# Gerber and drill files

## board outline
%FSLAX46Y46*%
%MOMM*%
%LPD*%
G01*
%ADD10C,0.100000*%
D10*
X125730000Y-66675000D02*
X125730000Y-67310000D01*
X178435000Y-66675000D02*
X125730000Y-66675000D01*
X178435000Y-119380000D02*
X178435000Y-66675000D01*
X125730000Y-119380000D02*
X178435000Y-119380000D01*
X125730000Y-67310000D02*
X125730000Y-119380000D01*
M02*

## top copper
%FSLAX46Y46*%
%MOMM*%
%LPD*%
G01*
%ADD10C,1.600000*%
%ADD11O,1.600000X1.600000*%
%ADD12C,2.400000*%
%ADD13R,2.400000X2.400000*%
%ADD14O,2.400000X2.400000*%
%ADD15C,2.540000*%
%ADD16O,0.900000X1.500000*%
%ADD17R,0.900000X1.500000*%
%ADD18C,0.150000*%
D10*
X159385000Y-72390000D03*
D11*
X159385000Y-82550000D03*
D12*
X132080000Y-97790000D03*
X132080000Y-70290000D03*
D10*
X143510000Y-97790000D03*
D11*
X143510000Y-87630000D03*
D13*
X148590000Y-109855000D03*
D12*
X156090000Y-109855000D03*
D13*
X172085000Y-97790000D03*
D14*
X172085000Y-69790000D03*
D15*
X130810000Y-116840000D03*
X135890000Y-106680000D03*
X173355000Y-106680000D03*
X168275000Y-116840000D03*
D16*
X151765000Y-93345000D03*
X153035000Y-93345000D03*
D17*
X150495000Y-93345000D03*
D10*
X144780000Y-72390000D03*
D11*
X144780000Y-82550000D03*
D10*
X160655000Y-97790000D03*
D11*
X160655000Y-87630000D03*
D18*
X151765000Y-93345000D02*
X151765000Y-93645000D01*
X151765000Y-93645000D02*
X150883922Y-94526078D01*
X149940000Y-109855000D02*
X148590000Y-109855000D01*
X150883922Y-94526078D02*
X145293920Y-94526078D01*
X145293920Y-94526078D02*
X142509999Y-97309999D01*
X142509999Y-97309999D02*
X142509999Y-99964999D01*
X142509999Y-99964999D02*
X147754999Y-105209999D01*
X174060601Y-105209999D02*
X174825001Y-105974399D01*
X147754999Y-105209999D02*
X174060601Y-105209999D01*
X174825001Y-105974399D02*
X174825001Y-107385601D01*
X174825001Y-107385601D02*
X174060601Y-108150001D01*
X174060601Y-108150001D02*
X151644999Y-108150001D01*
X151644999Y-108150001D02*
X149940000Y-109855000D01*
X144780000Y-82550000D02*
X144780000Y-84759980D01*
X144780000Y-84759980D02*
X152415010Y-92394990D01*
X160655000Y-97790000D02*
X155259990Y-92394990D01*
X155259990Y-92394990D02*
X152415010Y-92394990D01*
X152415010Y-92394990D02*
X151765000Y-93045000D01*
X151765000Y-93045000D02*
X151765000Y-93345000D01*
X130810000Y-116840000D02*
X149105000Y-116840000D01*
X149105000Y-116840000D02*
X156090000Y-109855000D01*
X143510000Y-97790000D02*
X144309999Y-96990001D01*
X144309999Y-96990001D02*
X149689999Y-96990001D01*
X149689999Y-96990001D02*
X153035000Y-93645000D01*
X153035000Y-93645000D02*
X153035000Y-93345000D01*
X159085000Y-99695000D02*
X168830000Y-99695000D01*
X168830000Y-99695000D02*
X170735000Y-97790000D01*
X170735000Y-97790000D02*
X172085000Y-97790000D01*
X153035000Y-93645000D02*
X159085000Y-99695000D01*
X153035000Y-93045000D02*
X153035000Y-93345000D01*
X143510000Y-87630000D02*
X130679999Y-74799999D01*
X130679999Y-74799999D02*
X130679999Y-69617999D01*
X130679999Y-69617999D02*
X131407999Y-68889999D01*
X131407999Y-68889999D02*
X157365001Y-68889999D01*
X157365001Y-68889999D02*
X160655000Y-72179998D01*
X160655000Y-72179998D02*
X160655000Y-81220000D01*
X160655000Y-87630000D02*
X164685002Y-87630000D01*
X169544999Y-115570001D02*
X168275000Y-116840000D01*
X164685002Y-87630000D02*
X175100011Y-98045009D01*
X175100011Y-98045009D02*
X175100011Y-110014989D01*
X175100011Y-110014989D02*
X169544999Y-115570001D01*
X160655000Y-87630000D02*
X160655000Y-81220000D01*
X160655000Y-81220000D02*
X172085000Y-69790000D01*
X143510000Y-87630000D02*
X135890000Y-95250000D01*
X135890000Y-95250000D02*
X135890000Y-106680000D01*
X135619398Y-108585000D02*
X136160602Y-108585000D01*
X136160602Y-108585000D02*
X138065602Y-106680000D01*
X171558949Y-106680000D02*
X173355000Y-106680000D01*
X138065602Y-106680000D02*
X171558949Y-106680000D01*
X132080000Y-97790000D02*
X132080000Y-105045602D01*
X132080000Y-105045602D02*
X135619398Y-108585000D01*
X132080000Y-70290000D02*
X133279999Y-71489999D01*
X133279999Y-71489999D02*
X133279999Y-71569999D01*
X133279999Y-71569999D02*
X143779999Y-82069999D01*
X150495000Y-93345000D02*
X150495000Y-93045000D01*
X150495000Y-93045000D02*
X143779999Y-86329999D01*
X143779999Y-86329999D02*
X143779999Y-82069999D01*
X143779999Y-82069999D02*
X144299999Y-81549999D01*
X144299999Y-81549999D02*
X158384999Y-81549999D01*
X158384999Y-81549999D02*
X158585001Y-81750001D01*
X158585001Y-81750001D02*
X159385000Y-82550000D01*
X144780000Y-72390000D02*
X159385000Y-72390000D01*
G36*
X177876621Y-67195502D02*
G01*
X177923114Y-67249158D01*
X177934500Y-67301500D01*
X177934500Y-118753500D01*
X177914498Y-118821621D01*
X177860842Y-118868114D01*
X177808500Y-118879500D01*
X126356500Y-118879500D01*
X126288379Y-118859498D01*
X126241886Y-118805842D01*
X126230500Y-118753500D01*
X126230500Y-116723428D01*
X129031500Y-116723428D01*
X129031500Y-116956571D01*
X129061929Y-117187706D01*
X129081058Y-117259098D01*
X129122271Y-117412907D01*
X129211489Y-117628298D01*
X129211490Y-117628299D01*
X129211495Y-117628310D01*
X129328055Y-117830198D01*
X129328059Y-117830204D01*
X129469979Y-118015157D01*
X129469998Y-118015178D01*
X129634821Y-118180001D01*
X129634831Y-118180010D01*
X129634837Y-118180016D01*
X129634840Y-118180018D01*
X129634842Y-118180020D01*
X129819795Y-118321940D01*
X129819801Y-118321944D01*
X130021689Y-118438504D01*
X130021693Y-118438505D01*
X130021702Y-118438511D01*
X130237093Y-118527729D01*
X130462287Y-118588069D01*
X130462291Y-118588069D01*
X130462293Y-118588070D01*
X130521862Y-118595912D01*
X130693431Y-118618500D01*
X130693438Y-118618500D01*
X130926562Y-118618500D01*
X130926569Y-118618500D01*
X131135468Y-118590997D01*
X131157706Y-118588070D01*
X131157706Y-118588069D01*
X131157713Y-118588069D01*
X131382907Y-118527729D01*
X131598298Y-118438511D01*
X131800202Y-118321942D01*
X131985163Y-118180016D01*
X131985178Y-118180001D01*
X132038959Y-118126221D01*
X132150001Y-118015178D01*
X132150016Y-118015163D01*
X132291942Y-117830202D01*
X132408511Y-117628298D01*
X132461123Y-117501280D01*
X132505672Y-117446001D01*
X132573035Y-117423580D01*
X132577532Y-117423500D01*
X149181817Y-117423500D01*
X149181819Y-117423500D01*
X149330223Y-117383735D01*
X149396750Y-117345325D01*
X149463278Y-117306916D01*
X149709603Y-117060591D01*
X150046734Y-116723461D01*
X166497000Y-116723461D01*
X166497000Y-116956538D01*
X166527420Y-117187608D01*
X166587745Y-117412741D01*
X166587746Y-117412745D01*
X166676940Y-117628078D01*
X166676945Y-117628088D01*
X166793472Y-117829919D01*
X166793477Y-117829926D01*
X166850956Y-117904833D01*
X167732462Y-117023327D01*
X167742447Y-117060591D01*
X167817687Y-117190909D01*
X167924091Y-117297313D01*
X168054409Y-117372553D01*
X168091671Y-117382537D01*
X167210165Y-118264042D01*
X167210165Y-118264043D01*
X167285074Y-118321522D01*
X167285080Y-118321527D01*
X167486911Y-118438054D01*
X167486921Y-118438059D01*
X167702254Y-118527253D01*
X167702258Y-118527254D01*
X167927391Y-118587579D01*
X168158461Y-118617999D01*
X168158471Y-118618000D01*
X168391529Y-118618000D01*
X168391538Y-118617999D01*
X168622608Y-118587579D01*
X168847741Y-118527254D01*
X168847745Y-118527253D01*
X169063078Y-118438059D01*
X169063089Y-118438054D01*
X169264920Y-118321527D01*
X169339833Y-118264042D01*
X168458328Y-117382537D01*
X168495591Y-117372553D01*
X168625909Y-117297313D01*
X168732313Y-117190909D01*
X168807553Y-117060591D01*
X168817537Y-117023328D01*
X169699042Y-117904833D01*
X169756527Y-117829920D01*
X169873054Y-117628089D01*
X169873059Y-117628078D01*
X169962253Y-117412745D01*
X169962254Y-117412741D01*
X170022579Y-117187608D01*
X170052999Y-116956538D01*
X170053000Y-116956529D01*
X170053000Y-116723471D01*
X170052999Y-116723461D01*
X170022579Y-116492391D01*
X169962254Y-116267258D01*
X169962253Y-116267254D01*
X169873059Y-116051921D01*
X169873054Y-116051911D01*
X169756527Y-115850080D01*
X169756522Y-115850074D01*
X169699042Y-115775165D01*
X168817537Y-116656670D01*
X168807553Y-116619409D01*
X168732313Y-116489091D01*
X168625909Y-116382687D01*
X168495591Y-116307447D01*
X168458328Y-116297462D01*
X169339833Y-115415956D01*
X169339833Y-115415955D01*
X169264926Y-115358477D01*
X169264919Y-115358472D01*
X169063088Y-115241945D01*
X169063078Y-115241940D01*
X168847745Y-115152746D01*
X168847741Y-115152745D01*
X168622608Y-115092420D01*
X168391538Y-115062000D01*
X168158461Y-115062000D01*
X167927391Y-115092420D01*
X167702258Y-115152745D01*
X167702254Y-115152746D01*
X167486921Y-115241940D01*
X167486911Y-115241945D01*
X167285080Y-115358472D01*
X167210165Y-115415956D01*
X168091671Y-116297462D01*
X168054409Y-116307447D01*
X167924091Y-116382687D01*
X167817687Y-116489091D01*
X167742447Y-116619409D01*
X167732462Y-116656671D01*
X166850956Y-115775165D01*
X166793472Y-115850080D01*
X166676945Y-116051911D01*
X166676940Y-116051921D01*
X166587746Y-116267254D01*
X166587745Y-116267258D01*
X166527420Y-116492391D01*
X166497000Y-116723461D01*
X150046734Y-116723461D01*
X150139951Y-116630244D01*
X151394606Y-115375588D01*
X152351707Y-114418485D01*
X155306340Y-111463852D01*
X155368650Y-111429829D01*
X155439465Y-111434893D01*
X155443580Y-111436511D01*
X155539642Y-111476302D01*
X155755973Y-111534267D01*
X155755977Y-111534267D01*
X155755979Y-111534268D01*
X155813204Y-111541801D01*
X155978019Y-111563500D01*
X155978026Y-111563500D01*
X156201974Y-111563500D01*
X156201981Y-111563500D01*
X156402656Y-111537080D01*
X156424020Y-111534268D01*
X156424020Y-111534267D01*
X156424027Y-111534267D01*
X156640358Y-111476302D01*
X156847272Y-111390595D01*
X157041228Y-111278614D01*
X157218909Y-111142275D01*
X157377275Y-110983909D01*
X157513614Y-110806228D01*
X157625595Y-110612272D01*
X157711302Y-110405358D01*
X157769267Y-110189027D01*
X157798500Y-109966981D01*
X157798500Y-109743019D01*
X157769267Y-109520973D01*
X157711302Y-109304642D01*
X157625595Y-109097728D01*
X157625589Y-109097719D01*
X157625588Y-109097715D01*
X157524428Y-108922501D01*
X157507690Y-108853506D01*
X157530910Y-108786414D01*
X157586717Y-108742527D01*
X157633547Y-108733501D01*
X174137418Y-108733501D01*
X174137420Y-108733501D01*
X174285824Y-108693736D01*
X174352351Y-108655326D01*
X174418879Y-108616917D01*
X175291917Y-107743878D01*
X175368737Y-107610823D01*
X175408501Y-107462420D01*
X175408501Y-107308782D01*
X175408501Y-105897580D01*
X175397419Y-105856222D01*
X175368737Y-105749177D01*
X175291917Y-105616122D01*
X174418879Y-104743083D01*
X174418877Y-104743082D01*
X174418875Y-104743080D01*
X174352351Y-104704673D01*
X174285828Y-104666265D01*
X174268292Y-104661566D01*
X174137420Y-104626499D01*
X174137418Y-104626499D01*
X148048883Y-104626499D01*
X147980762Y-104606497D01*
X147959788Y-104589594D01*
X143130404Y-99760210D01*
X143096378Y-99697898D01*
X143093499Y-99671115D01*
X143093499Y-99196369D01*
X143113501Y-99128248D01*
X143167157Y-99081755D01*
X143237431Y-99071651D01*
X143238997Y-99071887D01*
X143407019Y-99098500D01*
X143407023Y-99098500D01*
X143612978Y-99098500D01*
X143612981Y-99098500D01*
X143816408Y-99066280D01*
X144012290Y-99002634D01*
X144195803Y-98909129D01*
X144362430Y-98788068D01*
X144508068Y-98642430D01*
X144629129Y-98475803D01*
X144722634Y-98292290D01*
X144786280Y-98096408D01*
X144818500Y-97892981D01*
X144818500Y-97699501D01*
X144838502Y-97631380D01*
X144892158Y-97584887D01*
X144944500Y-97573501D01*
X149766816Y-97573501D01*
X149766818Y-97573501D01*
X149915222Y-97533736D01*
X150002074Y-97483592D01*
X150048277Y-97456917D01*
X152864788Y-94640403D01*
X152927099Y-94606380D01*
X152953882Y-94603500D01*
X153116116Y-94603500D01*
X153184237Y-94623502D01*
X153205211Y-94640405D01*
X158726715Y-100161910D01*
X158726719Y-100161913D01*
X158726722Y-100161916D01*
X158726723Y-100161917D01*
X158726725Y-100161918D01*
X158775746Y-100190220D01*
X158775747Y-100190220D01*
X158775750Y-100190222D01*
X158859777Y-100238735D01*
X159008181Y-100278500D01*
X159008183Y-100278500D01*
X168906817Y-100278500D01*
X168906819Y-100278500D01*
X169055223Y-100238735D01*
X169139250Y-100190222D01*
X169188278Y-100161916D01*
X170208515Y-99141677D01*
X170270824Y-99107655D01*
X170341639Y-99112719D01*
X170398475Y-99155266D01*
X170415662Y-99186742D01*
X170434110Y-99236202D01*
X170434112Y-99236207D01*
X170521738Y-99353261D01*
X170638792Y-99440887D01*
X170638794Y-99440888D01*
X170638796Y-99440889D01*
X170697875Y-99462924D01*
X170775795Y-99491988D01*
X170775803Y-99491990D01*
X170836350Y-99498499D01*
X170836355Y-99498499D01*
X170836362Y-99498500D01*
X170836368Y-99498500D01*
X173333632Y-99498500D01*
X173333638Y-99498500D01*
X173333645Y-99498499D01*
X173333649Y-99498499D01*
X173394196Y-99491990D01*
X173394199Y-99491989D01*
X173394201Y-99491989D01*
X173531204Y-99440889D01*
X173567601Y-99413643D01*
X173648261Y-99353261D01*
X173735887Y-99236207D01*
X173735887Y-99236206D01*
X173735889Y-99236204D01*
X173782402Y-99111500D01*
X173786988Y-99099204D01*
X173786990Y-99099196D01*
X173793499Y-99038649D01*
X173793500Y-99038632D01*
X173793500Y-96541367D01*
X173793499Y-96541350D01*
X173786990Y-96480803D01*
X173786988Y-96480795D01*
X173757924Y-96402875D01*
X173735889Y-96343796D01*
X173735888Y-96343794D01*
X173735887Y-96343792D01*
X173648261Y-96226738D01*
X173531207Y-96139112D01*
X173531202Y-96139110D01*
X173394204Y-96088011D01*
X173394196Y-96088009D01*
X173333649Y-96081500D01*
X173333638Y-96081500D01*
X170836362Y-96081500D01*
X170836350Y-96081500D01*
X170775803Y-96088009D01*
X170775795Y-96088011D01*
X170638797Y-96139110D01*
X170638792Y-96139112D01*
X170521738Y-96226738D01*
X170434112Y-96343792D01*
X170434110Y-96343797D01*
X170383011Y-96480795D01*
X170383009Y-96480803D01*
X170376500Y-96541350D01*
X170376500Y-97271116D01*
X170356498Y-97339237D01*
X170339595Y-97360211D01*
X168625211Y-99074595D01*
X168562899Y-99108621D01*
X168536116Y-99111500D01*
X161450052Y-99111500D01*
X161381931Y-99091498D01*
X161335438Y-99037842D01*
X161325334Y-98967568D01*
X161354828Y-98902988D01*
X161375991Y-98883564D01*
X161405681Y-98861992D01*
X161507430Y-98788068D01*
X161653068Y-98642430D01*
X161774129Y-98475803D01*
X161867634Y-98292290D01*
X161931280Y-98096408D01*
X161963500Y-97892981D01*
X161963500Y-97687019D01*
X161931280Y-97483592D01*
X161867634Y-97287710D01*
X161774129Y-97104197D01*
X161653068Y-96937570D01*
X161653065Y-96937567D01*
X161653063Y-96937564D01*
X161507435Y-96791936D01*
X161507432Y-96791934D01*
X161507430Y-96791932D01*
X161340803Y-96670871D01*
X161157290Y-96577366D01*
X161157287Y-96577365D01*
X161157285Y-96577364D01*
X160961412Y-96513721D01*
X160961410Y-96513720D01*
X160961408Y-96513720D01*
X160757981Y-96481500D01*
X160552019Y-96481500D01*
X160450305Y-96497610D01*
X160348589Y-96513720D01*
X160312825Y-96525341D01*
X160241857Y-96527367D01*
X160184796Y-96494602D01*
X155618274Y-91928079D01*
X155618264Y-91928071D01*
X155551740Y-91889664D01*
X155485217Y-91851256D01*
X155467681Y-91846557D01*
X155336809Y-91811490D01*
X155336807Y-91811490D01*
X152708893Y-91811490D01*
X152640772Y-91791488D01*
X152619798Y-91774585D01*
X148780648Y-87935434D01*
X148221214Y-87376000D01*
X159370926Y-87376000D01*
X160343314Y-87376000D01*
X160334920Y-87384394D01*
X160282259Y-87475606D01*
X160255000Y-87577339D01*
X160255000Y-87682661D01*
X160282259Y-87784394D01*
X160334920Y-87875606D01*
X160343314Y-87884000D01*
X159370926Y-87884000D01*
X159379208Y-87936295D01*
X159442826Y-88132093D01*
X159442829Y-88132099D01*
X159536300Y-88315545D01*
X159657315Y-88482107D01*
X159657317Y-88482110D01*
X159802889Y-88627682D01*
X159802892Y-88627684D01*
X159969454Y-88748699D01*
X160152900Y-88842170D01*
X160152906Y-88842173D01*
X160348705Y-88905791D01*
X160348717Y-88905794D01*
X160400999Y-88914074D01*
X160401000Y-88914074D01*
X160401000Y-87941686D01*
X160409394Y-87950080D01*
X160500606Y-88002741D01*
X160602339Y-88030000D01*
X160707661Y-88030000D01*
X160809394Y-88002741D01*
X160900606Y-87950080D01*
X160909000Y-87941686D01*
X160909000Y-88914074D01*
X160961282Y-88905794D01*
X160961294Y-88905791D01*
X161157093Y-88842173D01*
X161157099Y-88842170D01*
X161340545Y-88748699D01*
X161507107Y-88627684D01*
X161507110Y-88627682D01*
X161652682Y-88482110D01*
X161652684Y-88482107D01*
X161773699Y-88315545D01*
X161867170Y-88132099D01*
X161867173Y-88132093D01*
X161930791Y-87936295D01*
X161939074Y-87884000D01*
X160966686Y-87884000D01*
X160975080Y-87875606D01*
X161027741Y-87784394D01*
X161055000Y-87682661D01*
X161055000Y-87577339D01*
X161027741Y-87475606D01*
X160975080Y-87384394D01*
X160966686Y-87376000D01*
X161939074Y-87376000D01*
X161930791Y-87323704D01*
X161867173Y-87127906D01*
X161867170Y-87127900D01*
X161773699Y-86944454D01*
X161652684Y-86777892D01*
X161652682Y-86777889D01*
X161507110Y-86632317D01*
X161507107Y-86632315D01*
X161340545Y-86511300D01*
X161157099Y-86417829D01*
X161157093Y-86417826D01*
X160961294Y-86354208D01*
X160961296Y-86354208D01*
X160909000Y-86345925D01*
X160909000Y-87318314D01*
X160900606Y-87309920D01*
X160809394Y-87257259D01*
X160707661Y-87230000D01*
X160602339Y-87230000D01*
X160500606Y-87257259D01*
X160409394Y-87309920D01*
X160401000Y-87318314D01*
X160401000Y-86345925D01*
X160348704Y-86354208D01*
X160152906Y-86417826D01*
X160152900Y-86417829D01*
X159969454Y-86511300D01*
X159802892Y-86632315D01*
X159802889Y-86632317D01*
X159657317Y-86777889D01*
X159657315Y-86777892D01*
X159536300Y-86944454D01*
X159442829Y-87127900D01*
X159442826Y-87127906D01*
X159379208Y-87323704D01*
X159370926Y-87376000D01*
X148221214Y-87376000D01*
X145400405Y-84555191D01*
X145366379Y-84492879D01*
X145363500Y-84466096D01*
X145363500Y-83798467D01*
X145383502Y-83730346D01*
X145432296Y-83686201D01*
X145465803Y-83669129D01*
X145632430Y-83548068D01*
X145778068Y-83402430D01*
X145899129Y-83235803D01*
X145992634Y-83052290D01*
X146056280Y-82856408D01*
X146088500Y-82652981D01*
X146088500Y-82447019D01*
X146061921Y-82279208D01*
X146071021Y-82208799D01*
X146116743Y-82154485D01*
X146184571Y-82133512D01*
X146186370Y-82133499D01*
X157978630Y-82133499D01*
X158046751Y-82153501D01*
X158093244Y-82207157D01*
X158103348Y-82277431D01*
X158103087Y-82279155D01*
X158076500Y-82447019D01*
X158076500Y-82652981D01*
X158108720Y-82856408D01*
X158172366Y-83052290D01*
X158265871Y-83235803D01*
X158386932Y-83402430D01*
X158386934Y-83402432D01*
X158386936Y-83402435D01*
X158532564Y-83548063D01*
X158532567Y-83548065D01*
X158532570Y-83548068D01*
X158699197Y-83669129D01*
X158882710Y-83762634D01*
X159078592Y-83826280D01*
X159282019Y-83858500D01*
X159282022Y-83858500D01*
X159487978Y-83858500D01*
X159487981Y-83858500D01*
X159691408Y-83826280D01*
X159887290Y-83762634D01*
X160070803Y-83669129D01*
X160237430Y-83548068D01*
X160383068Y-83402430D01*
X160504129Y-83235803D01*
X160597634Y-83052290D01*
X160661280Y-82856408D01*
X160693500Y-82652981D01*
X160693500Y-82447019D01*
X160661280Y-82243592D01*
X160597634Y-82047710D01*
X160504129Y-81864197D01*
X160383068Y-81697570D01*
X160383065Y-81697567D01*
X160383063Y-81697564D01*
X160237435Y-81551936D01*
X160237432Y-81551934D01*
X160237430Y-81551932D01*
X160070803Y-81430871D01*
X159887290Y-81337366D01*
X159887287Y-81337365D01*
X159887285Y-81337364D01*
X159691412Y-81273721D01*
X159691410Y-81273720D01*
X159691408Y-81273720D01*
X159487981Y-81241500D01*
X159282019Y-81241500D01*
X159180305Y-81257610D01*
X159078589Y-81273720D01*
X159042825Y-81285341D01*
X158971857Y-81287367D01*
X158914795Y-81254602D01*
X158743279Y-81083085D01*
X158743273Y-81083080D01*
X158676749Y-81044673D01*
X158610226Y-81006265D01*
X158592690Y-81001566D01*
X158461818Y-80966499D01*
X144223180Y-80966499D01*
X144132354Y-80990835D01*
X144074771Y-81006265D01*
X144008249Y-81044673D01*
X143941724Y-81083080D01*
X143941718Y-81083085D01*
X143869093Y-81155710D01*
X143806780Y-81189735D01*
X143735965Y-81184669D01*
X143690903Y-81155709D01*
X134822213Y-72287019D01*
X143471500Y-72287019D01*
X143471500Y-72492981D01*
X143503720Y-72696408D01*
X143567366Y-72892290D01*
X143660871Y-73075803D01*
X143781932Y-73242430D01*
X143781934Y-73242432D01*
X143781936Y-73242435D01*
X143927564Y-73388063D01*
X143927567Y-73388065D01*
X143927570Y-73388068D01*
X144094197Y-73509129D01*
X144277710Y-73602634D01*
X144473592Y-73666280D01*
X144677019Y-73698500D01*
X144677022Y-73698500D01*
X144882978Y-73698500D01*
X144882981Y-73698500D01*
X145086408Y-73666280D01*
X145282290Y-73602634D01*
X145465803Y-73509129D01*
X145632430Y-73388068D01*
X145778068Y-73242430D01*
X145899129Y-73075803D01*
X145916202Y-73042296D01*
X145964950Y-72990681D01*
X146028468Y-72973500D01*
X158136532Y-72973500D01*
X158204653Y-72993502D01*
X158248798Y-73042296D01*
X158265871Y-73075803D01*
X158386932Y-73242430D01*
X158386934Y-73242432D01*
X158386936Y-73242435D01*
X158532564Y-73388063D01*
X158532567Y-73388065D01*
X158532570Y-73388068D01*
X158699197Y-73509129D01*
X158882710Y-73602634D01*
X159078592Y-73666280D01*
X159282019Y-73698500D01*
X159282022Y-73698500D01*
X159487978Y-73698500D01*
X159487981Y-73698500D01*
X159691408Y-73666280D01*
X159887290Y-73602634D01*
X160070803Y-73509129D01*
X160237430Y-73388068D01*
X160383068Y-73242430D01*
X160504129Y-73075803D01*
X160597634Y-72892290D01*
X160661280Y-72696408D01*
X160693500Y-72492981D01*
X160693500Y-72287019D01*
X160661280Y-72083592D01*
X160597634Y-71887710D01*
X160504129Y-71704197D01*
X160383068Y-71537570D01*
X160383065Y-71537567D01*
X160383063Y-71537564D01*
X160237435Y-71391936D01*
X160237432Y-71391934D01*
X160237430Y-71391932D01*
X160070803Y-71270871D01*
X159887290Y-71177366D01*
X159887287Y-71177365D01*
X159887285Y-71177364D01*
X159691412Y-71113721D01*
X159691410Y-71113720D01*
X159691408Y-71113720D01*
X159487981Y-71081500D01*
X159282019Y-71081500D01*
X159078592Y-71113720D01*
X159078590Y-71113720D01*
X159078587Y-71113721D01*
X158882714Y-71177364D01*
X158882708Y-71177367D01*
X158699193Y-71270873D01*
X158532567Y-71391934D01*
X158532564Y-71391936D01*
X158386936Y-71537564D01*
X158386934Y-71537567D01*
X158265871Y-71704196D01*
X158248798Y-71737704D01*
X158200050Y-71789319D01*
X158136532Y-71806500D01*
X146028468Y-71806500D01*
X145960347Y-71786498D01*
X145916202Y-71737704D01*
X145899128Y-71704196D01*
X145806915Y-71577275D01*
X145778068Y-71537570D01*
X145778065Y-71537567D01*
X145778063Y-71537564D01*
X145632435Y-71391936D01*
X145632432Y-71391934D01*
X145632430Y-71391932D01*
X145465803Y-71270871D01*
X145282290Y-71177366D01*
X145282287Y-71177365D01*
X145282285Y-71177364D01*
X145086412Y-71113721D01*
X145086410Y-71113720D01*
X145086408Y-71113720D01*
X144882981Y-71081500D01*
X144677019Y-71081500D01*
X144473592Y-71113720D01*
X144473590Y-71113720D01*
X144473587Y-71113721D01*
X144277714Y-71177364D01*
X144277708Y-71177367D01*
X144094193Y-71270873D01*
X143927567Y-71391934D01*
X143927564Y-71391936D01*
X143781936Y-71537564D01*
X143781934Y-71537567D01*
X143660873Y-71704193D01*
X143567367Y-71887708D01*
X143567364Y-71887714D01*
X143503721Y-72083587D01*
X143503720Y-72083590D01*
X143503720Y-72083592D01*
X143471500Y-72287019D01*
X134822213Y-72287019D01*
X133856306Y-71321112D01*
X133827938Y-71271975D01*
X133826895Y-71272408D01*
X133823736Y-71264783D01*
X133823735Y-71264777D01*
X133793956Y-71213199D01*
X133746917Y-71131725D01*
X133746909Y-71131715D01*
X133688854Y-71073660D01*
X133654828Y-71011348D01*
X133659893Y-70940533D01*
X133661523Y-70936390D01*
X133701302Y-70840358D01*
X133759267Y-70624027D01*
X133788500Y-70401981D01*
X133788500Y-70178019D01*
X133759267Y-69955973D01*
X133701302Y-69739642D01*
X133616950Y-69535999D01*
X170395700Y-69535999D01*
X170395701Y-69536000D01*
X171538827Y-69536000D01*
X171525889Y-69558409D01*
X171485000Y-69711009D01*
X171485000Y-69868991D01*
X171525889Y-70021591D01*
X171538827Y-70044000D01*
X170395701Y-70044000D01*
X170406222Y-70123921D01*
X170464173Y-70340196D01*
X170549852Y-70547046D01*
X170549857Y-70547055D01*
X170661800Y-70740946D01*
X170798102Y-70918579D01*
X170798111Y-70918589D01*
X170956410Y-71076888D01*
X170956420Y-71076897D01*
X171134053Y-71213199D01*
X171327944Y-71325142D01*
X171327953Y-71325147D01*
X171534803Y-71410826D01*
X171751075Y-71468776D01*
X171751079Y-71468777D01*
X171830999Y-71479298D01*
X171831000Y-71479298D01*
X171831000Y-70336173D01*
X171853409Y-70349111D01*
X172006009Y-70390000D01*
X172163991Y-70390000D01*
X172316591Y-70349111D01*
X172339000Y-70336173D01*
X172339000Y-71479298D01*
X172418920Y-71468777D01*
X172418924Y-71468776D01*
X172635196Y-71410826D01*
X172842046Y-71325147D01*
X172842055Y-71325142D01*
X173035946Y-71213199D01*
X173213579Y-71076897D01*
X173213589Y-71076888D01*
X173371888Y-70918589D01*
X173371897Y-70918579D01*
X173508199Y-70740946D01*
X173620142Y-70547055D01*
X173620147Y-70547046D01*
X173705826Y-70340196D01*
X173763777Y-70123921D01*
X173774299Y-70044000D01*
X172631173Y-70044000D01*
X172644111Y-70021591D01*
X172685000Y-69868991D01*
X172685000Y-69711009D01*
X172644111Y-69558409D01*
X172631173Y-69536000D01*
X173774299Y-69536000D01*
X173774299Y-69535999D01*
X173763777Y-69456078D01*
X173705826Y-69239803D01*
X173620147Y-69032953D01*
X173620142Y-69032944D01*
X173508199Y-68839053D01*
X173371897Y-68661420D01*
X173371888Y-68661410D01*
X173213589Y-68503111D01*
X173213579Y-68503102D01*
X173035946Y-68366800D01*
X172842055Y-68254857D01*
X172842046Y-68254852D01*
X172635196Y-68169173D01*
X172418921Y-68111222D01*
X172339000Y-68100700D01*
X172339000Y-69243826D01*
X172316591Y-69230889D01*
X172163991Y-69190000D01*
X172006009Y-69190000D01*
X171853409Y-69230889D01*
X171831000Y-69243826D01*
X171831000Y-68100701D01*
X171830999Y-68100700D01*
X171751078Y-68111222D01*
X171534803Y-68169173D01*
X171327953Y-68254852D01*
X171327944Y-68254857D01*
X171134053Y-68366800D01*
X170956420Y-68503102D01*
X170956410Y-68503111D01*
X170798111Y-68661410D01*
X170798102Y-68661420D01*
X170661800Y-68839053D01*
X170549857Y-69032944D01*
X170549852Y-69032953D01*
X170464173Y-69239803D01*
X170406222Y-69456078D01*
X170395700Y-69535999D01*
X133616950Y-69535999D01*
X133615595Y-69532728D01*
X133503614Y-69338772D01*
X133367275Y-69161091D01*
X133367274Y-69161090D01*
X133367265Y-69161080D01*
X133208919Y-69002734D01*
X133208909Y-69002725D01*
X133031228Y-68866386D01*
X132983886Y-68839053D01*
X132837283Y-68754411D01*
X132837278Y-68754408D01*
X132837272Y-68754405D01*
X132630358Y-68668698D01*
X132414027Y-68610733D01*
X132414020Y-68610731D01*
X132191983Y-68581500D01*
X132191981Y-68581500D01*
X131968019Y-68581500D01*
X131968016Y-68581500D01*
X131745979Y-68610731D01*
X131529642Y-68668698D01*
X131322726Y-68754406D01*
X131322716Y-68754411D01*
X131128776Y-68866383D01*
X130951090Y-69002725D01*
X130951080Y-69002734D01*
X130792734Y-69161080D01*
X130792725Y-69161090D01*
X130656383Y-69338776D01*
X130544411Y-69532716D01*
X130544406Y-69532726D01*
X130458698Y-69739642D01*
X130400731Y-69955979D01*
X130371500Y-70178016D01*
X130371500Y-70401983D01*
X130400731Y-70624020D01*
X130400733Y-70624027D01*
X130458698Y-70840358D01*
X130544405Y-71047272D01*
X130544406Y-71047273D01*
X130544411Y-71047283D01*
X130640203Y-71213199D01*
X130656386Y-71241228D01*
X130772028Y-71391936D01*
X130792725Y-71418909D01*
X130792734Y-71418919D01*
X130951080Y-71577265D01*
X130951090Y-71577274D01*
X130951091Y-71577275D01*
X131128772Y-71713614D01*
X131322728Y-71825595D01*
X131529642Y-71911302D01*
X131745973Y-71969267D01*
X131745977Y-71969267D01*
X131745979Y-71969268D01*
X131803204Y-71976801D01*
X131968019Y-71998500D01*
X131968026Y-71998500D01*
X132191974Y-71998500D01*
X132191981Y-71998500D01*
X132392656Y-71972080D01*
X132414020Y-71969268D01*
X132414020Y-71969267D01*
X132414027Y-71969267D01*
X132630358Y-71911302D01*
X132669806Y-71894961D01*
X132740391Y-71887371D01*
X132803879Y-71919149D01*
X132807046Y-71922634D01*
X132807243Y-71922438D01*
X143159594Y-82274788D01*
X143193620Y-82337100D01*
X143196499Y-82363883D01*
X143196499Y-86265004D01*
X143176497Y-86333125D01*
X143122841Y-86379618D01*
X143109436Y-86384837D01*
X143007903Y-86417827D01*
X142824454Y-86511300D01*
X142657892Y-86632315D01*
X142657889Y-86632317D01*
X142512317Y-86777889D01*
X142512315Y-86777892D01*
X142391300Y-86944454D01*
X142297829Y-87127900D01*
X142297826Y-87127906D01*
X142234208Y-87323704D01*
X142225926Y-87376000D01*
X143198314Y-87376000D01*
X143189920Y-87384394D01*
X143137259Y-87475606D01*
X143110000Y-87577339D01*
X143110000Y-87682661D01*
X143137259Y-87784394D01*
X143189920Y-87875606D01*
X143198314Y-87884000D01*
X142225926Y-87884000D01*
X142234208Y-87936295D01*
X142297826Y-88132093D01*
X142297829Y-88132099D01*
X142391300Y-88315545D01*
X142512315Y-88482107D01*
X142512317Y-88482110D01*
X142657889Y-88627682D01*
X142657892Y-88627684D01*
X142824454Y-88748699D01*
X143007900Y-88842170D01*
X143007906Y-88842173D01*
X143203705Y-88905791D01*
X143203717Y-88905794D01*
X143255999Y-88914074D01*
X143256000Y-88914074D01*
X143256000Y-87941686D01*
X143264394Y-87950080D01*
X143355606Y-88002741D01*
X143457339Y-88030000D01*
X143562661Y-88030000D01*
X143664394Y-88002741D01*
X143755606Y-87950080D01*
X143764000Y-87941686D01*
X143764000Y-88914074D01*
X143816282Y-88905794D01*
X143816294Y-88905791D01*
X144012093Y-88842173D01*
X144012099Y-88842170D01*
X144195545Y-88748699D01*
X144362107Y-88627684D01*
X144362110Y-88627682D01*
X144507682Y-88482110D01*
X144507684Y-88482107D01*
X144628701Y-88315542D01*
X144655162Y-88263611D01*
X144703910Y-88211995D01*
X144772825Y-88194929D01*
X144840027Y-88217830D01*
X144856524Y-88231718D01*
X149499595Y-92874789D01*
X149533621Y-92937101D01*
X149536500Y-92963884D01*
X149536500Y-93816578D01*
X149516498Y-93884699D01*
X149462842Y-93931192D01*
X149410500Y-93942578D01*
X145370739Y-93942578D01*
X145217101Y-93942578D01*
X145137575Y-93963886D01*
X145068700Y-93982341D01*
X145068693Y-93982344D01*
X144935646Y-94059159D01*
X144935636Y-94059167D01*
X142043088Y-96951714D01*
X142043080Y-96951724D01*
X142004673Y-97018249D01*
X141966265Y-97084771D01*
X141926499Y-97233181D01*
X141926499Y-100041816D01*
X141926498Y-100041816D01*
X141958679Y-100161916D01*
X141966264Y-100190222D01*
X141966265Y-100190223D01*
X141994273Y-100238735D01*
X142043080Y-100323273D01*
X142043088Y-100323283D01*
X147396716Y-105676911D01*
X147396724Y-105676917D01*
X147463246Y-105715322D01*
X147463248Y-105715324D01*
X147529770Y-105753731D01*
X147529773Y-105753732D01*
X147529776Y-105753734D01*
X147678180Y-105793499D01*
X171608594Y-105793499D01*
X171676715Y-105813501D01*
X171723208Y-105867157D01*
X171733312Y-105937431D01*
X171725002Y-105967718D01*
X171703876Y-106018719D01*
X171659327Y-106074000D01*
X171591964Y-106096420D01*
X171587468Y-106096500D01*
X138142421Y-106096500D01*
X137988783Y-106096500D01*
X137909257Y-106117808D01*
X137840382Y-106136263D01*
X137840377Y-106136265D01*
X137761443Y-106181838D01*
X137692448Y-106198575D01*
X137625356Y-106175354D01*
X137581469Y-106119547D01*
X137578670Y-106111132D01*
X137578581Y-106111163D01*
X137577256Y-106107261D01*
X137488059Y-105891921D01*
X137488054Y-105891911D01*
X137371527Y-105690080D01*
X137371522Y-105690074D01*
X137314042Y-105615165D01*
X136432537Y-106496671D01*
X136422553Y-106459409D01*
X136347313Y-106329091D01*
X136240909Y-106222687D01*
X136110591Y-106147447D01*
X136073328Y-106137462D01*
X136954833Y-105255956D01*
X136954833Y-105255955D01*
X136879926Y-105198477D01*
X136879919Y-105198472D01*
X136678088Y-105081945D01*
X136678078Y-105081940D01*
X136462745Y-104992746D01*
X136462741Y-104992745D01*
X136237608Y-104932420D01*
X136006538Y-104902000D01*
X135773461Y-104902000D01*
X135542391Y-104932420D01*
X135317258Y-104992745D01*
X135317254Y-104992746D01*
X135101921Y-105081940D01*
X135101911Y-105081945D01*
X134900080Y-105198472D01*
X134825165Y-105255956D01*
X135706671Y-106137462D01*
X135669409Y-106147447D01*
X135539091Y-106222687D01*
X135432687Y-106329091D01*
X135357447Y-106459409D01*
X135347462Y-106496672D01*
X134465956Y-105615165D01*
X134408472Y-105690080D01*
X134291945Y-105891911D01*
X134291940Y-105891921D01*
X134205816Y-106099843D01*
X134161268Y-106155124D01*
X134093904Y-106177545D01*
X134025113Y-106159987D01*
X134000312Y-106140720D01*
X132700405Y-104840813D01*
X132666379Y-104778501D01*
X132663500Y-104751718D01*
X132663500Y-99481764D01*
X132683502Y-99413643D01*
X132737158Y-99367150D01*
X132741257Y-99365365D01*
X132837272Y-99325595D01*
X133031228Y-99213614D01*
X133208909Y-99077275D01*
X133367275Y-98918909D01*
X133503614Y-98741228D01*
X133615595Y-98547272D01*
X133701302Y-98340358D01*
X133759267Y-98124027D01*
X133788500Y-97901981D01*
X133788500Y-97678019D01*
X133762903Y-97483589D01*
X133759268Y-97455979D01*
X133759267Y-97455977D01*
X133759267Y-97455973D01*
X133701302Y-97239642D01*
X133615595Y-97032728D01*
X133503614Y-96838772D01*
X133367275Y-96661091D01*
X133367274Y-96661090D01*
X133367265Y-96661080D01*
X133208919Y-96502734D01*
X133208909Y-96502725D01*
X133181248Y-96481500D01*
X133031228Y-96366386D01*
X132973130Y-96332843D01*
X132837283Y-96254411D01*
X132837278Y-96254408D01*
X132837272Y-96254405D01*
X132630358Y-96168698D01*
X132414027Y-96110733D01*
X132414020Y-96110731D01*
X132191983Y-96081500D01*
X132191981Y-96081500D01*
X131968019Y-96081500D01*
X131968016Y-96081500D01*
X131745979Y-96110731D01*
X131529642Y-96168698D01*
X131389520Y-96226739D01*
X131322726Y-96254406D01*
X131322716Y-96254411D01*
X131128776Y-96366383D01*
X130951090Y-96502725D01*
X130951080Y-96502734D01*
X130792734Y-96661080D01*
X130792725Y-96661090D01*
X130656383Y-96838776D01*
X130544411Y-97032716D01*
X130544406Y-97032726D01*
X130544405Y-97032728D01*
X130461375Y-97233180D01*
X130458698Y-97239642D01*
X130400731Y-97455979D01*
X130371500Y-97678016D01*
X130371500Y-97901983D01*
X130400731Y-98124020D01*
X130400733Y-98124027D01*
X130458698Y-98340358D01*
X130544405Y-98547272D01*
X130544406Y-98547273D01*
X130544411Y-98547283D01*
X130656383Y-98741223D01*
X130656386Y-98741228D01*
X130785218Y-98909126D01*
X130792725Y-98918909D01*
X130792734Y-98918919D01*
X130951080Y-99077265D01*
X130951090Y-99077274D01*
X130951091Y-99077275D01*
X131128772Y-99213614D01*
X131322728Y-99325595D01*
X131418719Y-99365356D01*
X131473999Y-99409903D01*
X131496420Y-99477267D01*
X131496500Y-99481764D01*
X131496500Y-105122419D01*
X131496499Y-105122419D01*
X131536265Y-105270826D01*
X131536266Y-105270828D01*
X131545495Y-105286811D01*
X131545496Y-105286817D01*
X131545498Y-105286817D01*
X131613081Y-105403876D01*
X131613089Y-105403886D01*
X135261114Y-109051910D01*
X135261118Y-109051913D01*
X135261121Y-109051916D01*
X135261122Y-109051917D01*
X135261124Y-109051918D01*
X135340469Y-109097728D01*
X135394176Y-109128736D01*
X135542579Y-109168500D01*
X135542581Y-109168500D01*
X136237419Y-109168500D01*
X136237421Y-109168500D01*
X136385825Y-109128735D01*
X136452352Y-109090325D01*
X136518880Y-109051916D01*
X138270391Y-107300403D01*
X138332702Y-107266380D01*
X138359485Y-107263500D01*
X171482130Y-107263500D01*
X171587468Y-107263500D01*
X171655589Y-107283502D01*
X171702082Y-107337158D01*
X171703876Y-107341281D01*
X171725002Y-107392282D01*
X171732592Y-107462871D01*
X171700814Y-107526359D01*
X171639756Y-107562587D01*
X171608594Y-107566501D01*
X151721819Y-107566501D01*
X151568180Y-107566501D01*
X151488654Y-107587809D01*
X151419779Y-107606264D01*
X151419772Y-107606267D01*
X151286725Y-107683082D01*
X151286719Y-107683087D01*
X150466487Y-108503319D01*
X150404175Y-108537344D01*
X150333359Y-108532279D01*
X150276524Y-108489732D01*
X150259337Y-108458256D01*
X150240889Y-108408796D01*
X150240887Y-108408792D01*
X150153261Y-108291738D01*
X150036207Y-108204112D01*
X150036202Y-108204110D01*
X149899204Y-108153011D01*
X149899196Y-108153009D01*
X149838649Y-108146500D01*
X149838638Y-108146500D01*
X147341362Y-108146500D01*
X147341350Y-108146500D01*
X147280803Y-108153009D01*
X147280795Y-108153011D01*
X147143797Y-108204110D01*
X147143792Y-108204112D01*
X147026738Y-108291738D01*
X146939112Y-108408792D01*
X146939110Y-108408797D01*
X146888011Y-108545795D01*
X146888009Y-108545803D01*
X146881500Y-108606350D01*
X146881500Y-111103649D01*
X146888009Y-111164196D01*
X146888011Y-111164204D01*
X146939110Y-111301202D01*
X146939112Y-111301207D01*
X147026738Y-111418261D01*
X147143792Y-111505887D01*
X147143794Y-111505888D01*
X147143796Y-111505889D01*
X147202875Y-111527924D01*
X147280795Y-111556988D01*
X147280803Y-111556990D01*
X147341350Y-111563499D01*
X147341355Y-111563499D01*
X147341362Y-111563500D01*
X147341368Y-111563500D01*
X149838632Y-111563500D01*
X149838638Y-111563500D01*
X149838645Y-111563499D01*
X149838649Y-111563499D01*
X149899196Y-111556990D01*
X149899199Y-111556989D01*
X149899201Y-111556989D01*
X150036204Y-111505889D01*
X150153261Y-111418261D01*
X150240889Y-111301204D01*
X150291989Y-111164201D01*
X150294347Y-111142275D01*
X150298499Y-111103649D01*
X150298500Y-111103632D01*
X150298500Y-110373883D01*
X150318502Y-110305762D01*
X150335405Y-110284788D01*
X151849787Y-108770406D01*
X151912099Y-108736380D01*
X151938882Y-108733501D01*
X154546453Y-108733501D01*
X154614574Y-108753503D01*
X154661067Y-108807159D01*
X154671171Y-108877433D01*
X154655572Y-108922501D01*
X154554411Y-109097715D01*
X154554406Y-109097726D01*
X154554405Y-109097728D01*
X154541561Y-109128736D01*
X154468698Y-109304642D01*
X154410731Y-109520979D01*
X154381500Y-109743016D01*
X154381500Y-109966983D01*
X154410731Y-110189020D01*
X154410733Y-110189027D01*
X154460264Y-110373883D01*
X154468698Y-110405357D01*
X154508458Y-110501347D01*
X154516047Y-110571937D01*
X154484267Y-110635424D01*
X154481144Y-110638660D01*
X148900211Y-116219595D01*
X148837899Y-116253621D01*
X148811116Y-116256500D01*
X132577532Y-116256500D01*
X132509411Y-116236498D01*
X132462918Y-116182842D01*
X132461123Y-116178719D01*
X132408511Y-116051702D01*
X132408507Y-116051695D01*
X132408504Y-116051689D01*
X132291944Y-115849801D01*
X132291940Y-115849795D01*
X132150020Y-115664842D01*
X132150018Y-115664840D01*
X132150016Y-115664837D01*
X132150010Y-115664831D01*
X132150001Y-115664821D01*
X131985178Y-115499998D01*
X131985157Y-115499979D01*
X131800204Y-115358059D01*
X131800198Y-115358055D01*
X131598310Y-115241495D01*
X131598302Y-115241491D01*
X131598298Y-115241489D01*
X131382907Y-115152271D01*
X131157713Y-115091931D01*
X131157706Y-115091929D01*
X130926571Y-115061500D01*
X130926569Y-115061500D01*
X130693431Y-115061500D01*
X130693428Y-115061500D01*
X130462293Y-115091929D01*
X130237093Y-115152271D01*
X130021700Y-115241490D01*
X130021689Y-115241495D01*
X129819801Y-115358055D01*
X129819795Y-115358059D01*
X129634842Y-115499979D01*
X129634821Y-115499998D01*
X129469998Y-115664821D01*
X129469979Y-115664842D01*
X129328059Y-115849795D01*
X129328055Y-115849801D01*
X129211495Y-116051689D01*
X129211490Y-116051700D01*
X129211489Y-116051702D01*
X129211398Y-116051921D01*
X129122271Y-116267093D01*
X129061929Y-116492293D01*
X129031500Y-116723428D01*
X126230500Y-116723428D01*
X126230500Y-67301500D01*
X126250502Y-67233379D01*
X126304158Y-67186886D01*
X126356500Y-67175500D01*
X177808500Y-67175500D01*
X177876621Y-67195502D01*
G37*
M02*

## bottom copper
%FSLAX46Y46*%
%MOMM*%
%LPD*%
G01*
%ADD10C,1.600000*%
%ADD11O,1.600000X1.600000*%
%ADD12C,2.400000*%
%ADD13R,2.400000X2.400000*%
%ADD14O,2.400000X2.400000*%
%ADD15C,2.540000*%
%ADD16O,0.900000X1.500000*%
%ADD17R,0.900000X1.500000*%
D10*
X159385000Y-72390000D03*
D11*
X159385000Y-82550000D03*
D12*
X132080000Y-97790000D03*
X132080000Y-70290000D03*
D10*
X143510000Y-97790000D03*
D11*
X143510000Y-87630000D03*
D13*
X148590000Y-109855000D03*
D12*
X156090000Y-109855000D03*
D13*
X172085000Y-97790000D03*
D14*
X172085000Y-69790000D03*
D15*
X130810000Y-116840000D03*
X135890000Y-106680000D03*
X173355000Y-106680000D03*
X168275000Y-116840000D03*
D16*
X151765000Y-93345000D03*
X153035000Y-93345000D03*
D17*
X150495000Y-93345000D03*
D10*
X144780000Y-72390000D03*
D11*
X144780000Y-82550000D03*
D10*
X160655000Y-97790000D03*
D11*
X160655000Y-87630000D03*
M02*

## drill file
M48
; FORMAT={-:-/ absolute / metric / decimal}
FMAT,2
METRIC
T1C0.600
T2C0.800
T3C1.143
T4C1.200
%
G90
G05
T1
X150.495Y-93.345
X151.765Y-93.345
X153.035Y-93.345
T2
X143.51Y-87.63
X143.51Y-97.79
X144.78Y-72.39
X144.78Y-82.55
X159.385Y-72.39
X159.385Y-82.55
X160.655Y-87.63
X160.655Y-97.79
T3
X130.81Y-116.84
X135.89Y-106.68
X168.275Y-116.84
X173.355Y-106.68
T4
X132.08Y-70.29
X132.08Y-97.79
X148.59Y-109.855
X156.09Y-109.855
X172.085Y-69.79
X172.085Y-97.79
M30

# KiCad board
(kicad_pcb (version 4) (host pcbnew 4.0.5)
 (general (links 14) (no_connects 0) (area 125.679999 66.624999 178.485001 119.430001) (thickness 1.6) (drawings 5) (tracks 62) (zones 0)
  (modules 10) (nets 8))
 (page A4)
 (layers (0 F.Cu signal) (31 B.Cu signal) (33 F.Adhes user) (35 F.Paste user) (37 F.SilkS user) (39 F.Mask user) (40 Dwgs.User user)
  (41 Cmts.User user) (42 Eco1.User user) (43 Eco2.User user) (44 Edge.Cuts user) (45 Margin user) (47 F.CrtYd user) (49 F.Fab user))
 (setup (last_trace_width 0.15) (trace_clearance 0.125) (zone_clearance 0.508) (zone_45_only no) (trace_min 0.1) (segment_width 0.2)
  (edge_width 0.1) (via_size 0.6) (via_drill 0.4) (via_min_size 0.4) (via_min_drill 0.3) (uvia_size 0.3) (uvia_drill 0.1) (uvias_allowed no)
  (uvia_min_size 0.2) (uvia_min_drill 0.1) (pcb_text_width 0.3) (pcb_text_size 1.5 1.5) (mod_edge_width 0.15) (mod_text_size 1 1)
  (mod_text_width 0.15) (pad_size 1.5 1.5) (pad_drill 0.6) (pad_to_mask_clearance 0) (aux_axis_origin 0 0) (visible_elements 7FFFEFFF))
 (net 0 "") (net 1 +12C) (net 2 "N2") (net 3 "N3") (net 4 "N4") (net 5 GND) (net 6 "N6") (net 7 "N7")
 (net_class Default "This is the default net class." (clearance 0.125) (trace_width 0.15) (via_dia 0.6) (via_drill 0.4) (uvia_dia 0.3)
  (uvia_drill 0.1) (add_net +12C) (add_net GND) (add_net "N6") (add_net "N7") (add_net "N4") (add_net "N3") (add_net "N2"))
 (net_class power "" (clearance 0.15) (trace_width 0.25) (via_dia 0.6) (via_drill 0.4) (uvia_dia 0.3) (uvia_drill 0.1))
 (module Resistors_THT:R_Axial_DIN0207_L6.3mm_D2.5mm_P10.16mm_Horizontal (layer F.Cu) (at 159.385 72.39 270)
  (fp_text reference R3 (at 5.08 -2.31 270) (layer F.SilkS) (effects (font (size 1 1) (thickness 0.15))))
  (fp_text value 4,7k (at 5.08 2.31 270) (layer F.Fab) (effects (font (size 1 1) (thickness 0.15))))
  (pad 1 thru_hole circle (at 0 0 270) (size 1.6 1.6) (drill 0.8) (layers *.Cu *.Mask) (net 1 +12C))
  (pad 2 thru_hole oval (at 10.16 0 270) (size 1.6 1.6) (drill 0.8) (layers *.Cu *.Mask) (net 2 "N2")))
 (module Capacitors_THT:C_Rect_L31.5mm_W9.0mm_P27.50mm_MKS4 (layer F.Cu) (at 132.08 97.79 90)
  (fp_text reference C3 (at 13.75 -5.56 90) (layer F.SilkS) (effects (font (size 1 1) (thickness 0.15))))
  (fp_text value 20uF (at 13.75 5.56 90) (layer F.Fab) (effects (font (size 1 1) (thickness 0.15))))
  (pad 1 thru_hole circle (at 0 0 90) (size 2.4 2.4) (drill 1.2) (layers *.Cu *.Mask) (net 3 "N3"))
  (pad 2 thru_hole circle (at 27.5 0 90) (size 2.4 2.4) (drill 1.2) (layers *.Cu *.Mask) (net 2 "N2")))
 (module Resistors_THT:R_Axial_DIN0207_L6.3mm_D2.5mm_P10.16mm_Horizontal (layer F.Cu) (at 143.51 97.79 90)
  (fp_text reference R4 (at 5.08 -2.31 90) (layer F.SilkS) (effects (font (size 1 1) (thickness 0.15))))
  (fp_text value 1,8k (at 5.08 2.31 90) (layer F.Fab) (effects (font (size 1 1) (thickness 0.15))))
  (pad 1 thru_hole circle (at 0 0 90) (size 1.6 1.6) (drill 0.8) (layers *.Cu *.Mask) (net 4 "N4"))
  (pad 2 thru_hole oval (at 10.16 0 90) (size 1.6 1.6) (drill 0.8) (layers *.Cu *.Mask) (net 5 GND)))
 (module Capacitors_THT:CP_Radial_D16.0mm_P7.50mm (layer F.Cu) (at 148.59 109.855)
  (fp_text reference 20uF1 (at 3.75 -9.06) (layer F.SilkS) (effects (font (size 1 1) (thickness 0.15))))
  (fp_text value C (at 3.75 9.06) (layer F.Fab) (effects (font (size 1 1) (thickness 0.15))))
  (pad 1 thru_hole rect (at 0 0) (size 2.4 2.4) (drill 1.2) (layers *.Cu *.Mask) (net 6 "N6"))
  (pad 2 thru_hole circle (at 7.5 0) (size 2.4 2.4) (drill 1.2) (layers *.Cu *.Mask) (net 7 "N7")))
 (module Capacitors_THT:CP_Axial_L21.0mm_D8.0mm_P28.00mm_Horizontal (layer F.Cu) (at 172.085 97.79 90)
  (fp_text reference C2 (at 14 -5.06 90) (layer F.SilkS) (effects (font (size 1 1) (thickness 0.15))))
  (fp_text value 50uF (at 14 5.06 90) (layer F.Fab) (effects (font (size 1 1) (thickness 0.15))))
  (pad 1 thru_hole rect (at 0 0 90) (size 2.4 2.4) (drill 1.2) (layers *.Cu *.Mask) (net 4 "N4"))
  (pad 2 thru_hole oval (at 28 0 90) (size 2.4 2.4) (drill 1.2) (layers *.Cu *.Mask) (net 5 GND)))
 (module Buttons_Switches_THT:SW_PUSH (layer F.Cu) (at 133.35 111.76 90)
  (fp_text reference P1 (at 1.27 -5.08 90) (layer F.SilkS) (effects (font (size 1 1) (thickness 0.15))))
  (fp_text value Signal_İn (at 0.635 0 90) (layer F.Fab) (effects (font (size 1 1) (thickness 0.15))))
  (pad 1 thru_hole circle (at -5.08 -2.54 90) (size 2.54 2.54) (drill 1.143) (layers *.Cu *.Mask) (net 7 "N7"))
  (pad 2 thru_hole circle (at 5.08 2.54 90) (size 2.54 2.54) (drill 1.143) (layers *.Cu *.Mask) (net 5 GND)))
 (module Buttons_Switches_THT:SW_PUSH (layer F.Cu) (at 170.815 111.76 270)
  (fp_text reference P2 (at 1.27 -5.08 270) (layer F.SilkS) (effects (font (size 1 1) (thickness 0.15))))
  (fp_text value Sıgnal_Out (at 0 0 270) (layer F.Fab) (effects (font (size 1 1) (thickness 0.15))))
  (pad 1 thru_hole circle (at -5.08 -2.54 270) (size 2.54 2.54) (drill 1.143) (layers *.Cu *.Mask) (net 3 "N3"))
  (pad 2 thru_hole circle (at 5.08 2.54 270) (size 2.54 2.54) (drill 1.143) (layers *.Cu *.Mask) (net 5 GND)))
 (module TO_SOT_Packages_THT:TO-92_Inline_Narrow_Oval (layer F.Cu) (at 150.495 93.345)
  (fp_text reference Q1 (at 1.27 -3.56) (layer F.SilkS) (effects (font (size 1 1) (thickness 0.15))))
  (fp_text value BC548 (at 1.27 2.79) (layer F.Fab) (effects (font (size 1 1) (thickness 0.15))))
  (pad 2 thru_hole oval (at 1.27 0 180) (size 0.9 1.5) (drill 0.6) (layers *.Cu *.Mask) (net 6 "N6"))
  (pad 3 thru_hole oval (at 2.54 0 180) (size 0.9 1.5) (drill 0.6) (layers *.Cu *.Mask) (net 4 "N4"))
  (pad 1 thru_hole rect (at 0 0 180) (size 0.9 1.5) (drill 0.6) (layers *.Cu *.Mask) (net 2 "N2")))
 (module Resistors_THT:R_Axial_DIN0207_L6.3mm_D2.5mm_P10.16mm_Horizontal (layer F.Cu) (at 144.78 72.39 270)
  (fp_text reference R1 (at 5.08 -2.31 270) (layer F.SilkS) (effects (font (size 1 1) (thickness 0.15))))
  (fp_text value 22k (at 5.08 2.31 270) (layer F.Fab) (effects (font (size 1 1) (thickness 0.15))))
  (pad 1 thru_hole circle (at 0 0 270) (size 1.6 1.6) (drill 0.8) (layers *.Cu *.Mask) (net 1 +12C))
  (pad 2 thru_hole oval (at 10.16 0 270) (size 1.6 1.6) (drill 0.8) (layers *.Cu *.Mask) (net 6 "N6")))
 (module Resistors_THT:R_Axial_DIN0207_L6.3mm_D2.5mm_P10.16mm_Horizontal (layer F.Cu) (at 160.655 97.79 90)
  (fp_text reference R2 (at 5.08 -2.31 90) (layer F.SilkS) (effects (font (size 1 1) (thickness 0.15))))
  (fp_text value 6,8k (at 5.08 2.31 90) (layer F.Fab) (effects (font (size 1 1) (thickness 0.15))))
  (pad 1 thru_hole circle (at 0 0 90) (size 1.6 1.6) (drill 0.8) (layers *.Cu *.Mask) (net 6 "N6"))
  (pad 2 thru_hole oval (at 10.16 0 90) (size 1.6 1.6) (drill 0.8) (layers *.Cu *.Mask) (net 5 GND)))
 (gr_line (start 125.73 66.675) (end 125.73 67.31) (layer Edge.Cuts) (width 0.1))
 (gr_line (start 178.435 66.675) (end 125.73 66.675) (layer Edge.Cuts) (width 0.1))
 (gr_line (start 178.435 119.38) (end 178.435 66.675) (layer Edge.Cuts) (width 0.1))
 (gr_line (start 125.73 119.38) (end 178.435 119.38) (layer Edge.Cuts) (width 0.1))
 (gr_line (start 125.73 67.31) (end 125.73 119.38) (layer Edge.Cuts) (width 0.1))
 (segment (start 151.765 93.345) (end 151.765 93.645) (width 0.15) (layer F.Cu) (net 6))
 (segment (start 151.765 93.645) (end 150.883922 94.526078) (width 0.15) (layer F.Cu) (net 6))
 (segment (start 149.94 109.855) (end 148.59 109.855) (width 0.15) (layer F.Cu) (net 6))
 (segment (start 150.883922 94.526078) (end 145.29392 94.526078) (width 0.15) (layer F.Cu) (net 6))
 (segment (start 145.29392 94.526078) (end 142.509999 97.309999) (width 0.15) (layer F.Cu) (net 6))
 (segment (start 142.509999 97.309999) (end 142.509999 99.964999) (width 0.15) (layer F.Cu) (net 6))
 (segment (start 142.509999 99.964999) (end 147.754999 105.209999) (width 0.15) (layer F.Cu) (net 6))
 (segment (start 174.060601 105.209999) (end 174.825001 105.974399) (width 0.15) (layer F.Cu) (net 6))
 (segment (start 147.754999 105.209999) (end 174.060601 105.209999) (width 0.15) (layer F.Cu) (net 6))
 (segment (start 174.825001 105.974399) (end 174.825001 107.385601) (width 0.15) (layer F.Cu) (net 6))
 (segment (start 174.825001 107.385601) (end 174.060601 108.150001) (width 0.15) (layer F.Cu) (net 6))
 (segment (start 174.060601 108.150001) (end 151.644999 108.150001) (width 0.15) (layer F.Cu) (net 6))
 (segment (start 151.644999 108.150001) (end 149.94 109.855) (width 0.15) (layer F.Cu) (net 6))
 (segment (start 144.78 82.55) (end 144.78 84.75998) (width 0.15) (layer F.Cu) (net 6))
 (segment (start 144.78 84.75998) (end 152.41501 92.39499) (width 0.15) (layer F.Cu) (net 6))
 (segment (start 160.655 97.79) (end 155.25999 92.39499) (width 0.15) (layer F.Cu) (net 6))
 (segment (start 155.25999 92.39499) (end 152.41501 92.39499) (width 0.15) (layer F.Cu) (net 6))
 (segment (start 152.41501 92.39499) (end 151.765 93.045) (width 0.15) (layer F.Cu) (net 6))
 (segment (start 151.765 93.045) (end 151.765 93.345) (width 0.15) (layer F.Cu) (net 6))
 (segment (start 130.81 116.84) (end 149.105 116.84) (width 0.15) (layer F.Cu) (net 7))
 (segment (start 149.105 116.84) (end 156.09 109.855) (width 0.15) (layer F.Cu) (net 7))
 (segment (start 143.51 97.79) (end 144.309999 96.990001) (width 0.15) (layer F.Cu) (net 4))
 (segment (start 144.309999 96.990001) (end 149.689999 96.990001) (width 0.15) (layer F.Cu) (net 4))
 (segment (start 149.689999 96.990001) (end 153.035 93.645) (width 0.15) (layer F.Cu) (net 4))
 (segment (start 153.035 93.645) (end 153.035 93.345) (width 0.15) (layer F.Cu) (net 4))
 (segment (start 159.085 99.695) (end 168.83 99.695) (width 0.15) (layer F.Cu) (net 4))
 (segment (start 168.83 99.695) (end 170.735 97.79) (width 0.15) (layer F.Cu) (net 4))
 (segment (start 170.735 97.79) (end 172.085 97.79) (width 0.15) (layer F.Cu) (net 4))
 (segment (start 153.035 93.645) (end 159.085 99.695) (width 0.15) (layer F.Cu) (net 4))
 (segment (start 153.035 93.045) (end 153.035 93.345) (width 0.15) (layer F.Cu) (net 4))
 (segment (start 143.51 87.63) (end 130.679999 74.799999) (width 0.15) (layer F.Cu) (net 5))
 (segment (start 130.679999 74.799999) (end 130.679999 69.617999) (width 0.15) (layer F.Cu) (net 5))
 (segment (start 130.679999 69.617999) (end 131.407999 68.889999) (width 0.15) (layer F.Cu) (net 5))
 (segment (start 131.407999 68.889999) (end 157.365001 68.889999) (width 0.15) (layer F.Cu) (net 5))
 (segment (start 157.365001 68.889999) (end 160.655 72.179998) (width 0.15) (layer F.Cu) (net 5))
 (segment (start 160.655 72.179998) (end 160.655 81.22) (width 0.15) (layer F.Cu) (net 5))
 (segment (start 160.655 87.63) (end 164.685002 87.63) (width 0.15) (layer F.Cu) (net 5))
 (segment (start 169.544999 115.570001) (end 168.275 116.84) (width 0.15) (layer F.Cu) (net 5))
 (segment (start 164.685002 87.63) (end 175.100011 98.045009) (width 0.15) (layer F.Cu) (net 5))
 (segment (start 175.100011 98.045009) (end 175.100011 110.014989) (width 0.15) (layer F.Cu) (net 5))
 (segment (start 175.100011 110.014989) (end 169.544999 115.570001) (width 0.15) (layer F.Cu) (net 5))
 (segment (start 160.655 87.63) (end 160.655 81.22) (width 0.15) (layer F.Cu) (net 5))
 (segment (start 160.655 81.22) (end 172.085 69.79) (width 0.15) (layer F.Cu) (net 5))
 (segment (start 143.51 87.63) (end 135.89 95.25) (width 0.15) (layer F.Cu) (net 5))
 (segment (start 135.89 95.25) (end 135.89 106.68) (width 0.15) (layer F.Cu) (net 5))
 (segment (start 135.619398 108.585) (end 136.160602 108.585) (width 0.15) (layer F.Cu) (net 3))
 (segment (start 136.160602 108.585) (end 138.065602 106.68) (width 0.15) (layer F.Cu) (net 3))
 (segment (start 171.558949 106.68) (end 173.355 106.68) (width 0.15) (layer F.Cu) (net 3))
 (segment (start 138.065602 106.68) (end 171.558949 106.68) (width 0.15) (layer F.Cu) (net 3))
 (segment (start 132.08 97.79) (end 132.08 105.045602) (width 0.15) (layer F.Cu) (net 3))
 (segment (start 132.08 105.045602) (end 135.619398 108.585) (width 0.15) (layer F.Cu) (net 3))
 (segment (start 132.08 70.29) (end 133.279999 71.489999) (width 0.15) (layer F.Cu) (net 2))
 (segment (start 133.279999 71.489999) (end 133.279999 71.569999) (width 0.15) (layer F.Cu) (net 2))
 (segment (start 133.279999 71.569999) (end 143.779999 82.069999) (width 0.15) (layer F.Cu) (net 2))
 (segment (start 150.495 93.345) (end 150.495 93.045) (width 0.15) (layer F.Cu) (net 2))
 (segment (start 150.495 93.045) (end 143.779999 86.329999) (width 0.15) (layer F.Cu) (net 2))
 (segment (start 143.779999 86.329999) (end 143.779999 82.069999) (width 0.15) (layer F.Cu) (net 2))
 (segment (start 143.779999 82.069999) (end 144.299999 81.549999) (width 0.15) (layer F.Cu) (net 2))
 (segment (start 144.299999 81.549999) (end 158.384999 81.549999) (width 0.15) (layer F.Cu) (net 2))
 (segment (start 158.384999 81.549999) (end 158.585001 81.750001) (width 0.15) (layer F.Cu) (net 2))
 (segment (start 158.585001 81.750001) (end 159.385 82.55) (width 0.15) (layer F.Cu) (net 2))
 (segment (start 144.78 72.39) (end 159.385 72.39) (width 0.15) (layer F.Cu) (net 1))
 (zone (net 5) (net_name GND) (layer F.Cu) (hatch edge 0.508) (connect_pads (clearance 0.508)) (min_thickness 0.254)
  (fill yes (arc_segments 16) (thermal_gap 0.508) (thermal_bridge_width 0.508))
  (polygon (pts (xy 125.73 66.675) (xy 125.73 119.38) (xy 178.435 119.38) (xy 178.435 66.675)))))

